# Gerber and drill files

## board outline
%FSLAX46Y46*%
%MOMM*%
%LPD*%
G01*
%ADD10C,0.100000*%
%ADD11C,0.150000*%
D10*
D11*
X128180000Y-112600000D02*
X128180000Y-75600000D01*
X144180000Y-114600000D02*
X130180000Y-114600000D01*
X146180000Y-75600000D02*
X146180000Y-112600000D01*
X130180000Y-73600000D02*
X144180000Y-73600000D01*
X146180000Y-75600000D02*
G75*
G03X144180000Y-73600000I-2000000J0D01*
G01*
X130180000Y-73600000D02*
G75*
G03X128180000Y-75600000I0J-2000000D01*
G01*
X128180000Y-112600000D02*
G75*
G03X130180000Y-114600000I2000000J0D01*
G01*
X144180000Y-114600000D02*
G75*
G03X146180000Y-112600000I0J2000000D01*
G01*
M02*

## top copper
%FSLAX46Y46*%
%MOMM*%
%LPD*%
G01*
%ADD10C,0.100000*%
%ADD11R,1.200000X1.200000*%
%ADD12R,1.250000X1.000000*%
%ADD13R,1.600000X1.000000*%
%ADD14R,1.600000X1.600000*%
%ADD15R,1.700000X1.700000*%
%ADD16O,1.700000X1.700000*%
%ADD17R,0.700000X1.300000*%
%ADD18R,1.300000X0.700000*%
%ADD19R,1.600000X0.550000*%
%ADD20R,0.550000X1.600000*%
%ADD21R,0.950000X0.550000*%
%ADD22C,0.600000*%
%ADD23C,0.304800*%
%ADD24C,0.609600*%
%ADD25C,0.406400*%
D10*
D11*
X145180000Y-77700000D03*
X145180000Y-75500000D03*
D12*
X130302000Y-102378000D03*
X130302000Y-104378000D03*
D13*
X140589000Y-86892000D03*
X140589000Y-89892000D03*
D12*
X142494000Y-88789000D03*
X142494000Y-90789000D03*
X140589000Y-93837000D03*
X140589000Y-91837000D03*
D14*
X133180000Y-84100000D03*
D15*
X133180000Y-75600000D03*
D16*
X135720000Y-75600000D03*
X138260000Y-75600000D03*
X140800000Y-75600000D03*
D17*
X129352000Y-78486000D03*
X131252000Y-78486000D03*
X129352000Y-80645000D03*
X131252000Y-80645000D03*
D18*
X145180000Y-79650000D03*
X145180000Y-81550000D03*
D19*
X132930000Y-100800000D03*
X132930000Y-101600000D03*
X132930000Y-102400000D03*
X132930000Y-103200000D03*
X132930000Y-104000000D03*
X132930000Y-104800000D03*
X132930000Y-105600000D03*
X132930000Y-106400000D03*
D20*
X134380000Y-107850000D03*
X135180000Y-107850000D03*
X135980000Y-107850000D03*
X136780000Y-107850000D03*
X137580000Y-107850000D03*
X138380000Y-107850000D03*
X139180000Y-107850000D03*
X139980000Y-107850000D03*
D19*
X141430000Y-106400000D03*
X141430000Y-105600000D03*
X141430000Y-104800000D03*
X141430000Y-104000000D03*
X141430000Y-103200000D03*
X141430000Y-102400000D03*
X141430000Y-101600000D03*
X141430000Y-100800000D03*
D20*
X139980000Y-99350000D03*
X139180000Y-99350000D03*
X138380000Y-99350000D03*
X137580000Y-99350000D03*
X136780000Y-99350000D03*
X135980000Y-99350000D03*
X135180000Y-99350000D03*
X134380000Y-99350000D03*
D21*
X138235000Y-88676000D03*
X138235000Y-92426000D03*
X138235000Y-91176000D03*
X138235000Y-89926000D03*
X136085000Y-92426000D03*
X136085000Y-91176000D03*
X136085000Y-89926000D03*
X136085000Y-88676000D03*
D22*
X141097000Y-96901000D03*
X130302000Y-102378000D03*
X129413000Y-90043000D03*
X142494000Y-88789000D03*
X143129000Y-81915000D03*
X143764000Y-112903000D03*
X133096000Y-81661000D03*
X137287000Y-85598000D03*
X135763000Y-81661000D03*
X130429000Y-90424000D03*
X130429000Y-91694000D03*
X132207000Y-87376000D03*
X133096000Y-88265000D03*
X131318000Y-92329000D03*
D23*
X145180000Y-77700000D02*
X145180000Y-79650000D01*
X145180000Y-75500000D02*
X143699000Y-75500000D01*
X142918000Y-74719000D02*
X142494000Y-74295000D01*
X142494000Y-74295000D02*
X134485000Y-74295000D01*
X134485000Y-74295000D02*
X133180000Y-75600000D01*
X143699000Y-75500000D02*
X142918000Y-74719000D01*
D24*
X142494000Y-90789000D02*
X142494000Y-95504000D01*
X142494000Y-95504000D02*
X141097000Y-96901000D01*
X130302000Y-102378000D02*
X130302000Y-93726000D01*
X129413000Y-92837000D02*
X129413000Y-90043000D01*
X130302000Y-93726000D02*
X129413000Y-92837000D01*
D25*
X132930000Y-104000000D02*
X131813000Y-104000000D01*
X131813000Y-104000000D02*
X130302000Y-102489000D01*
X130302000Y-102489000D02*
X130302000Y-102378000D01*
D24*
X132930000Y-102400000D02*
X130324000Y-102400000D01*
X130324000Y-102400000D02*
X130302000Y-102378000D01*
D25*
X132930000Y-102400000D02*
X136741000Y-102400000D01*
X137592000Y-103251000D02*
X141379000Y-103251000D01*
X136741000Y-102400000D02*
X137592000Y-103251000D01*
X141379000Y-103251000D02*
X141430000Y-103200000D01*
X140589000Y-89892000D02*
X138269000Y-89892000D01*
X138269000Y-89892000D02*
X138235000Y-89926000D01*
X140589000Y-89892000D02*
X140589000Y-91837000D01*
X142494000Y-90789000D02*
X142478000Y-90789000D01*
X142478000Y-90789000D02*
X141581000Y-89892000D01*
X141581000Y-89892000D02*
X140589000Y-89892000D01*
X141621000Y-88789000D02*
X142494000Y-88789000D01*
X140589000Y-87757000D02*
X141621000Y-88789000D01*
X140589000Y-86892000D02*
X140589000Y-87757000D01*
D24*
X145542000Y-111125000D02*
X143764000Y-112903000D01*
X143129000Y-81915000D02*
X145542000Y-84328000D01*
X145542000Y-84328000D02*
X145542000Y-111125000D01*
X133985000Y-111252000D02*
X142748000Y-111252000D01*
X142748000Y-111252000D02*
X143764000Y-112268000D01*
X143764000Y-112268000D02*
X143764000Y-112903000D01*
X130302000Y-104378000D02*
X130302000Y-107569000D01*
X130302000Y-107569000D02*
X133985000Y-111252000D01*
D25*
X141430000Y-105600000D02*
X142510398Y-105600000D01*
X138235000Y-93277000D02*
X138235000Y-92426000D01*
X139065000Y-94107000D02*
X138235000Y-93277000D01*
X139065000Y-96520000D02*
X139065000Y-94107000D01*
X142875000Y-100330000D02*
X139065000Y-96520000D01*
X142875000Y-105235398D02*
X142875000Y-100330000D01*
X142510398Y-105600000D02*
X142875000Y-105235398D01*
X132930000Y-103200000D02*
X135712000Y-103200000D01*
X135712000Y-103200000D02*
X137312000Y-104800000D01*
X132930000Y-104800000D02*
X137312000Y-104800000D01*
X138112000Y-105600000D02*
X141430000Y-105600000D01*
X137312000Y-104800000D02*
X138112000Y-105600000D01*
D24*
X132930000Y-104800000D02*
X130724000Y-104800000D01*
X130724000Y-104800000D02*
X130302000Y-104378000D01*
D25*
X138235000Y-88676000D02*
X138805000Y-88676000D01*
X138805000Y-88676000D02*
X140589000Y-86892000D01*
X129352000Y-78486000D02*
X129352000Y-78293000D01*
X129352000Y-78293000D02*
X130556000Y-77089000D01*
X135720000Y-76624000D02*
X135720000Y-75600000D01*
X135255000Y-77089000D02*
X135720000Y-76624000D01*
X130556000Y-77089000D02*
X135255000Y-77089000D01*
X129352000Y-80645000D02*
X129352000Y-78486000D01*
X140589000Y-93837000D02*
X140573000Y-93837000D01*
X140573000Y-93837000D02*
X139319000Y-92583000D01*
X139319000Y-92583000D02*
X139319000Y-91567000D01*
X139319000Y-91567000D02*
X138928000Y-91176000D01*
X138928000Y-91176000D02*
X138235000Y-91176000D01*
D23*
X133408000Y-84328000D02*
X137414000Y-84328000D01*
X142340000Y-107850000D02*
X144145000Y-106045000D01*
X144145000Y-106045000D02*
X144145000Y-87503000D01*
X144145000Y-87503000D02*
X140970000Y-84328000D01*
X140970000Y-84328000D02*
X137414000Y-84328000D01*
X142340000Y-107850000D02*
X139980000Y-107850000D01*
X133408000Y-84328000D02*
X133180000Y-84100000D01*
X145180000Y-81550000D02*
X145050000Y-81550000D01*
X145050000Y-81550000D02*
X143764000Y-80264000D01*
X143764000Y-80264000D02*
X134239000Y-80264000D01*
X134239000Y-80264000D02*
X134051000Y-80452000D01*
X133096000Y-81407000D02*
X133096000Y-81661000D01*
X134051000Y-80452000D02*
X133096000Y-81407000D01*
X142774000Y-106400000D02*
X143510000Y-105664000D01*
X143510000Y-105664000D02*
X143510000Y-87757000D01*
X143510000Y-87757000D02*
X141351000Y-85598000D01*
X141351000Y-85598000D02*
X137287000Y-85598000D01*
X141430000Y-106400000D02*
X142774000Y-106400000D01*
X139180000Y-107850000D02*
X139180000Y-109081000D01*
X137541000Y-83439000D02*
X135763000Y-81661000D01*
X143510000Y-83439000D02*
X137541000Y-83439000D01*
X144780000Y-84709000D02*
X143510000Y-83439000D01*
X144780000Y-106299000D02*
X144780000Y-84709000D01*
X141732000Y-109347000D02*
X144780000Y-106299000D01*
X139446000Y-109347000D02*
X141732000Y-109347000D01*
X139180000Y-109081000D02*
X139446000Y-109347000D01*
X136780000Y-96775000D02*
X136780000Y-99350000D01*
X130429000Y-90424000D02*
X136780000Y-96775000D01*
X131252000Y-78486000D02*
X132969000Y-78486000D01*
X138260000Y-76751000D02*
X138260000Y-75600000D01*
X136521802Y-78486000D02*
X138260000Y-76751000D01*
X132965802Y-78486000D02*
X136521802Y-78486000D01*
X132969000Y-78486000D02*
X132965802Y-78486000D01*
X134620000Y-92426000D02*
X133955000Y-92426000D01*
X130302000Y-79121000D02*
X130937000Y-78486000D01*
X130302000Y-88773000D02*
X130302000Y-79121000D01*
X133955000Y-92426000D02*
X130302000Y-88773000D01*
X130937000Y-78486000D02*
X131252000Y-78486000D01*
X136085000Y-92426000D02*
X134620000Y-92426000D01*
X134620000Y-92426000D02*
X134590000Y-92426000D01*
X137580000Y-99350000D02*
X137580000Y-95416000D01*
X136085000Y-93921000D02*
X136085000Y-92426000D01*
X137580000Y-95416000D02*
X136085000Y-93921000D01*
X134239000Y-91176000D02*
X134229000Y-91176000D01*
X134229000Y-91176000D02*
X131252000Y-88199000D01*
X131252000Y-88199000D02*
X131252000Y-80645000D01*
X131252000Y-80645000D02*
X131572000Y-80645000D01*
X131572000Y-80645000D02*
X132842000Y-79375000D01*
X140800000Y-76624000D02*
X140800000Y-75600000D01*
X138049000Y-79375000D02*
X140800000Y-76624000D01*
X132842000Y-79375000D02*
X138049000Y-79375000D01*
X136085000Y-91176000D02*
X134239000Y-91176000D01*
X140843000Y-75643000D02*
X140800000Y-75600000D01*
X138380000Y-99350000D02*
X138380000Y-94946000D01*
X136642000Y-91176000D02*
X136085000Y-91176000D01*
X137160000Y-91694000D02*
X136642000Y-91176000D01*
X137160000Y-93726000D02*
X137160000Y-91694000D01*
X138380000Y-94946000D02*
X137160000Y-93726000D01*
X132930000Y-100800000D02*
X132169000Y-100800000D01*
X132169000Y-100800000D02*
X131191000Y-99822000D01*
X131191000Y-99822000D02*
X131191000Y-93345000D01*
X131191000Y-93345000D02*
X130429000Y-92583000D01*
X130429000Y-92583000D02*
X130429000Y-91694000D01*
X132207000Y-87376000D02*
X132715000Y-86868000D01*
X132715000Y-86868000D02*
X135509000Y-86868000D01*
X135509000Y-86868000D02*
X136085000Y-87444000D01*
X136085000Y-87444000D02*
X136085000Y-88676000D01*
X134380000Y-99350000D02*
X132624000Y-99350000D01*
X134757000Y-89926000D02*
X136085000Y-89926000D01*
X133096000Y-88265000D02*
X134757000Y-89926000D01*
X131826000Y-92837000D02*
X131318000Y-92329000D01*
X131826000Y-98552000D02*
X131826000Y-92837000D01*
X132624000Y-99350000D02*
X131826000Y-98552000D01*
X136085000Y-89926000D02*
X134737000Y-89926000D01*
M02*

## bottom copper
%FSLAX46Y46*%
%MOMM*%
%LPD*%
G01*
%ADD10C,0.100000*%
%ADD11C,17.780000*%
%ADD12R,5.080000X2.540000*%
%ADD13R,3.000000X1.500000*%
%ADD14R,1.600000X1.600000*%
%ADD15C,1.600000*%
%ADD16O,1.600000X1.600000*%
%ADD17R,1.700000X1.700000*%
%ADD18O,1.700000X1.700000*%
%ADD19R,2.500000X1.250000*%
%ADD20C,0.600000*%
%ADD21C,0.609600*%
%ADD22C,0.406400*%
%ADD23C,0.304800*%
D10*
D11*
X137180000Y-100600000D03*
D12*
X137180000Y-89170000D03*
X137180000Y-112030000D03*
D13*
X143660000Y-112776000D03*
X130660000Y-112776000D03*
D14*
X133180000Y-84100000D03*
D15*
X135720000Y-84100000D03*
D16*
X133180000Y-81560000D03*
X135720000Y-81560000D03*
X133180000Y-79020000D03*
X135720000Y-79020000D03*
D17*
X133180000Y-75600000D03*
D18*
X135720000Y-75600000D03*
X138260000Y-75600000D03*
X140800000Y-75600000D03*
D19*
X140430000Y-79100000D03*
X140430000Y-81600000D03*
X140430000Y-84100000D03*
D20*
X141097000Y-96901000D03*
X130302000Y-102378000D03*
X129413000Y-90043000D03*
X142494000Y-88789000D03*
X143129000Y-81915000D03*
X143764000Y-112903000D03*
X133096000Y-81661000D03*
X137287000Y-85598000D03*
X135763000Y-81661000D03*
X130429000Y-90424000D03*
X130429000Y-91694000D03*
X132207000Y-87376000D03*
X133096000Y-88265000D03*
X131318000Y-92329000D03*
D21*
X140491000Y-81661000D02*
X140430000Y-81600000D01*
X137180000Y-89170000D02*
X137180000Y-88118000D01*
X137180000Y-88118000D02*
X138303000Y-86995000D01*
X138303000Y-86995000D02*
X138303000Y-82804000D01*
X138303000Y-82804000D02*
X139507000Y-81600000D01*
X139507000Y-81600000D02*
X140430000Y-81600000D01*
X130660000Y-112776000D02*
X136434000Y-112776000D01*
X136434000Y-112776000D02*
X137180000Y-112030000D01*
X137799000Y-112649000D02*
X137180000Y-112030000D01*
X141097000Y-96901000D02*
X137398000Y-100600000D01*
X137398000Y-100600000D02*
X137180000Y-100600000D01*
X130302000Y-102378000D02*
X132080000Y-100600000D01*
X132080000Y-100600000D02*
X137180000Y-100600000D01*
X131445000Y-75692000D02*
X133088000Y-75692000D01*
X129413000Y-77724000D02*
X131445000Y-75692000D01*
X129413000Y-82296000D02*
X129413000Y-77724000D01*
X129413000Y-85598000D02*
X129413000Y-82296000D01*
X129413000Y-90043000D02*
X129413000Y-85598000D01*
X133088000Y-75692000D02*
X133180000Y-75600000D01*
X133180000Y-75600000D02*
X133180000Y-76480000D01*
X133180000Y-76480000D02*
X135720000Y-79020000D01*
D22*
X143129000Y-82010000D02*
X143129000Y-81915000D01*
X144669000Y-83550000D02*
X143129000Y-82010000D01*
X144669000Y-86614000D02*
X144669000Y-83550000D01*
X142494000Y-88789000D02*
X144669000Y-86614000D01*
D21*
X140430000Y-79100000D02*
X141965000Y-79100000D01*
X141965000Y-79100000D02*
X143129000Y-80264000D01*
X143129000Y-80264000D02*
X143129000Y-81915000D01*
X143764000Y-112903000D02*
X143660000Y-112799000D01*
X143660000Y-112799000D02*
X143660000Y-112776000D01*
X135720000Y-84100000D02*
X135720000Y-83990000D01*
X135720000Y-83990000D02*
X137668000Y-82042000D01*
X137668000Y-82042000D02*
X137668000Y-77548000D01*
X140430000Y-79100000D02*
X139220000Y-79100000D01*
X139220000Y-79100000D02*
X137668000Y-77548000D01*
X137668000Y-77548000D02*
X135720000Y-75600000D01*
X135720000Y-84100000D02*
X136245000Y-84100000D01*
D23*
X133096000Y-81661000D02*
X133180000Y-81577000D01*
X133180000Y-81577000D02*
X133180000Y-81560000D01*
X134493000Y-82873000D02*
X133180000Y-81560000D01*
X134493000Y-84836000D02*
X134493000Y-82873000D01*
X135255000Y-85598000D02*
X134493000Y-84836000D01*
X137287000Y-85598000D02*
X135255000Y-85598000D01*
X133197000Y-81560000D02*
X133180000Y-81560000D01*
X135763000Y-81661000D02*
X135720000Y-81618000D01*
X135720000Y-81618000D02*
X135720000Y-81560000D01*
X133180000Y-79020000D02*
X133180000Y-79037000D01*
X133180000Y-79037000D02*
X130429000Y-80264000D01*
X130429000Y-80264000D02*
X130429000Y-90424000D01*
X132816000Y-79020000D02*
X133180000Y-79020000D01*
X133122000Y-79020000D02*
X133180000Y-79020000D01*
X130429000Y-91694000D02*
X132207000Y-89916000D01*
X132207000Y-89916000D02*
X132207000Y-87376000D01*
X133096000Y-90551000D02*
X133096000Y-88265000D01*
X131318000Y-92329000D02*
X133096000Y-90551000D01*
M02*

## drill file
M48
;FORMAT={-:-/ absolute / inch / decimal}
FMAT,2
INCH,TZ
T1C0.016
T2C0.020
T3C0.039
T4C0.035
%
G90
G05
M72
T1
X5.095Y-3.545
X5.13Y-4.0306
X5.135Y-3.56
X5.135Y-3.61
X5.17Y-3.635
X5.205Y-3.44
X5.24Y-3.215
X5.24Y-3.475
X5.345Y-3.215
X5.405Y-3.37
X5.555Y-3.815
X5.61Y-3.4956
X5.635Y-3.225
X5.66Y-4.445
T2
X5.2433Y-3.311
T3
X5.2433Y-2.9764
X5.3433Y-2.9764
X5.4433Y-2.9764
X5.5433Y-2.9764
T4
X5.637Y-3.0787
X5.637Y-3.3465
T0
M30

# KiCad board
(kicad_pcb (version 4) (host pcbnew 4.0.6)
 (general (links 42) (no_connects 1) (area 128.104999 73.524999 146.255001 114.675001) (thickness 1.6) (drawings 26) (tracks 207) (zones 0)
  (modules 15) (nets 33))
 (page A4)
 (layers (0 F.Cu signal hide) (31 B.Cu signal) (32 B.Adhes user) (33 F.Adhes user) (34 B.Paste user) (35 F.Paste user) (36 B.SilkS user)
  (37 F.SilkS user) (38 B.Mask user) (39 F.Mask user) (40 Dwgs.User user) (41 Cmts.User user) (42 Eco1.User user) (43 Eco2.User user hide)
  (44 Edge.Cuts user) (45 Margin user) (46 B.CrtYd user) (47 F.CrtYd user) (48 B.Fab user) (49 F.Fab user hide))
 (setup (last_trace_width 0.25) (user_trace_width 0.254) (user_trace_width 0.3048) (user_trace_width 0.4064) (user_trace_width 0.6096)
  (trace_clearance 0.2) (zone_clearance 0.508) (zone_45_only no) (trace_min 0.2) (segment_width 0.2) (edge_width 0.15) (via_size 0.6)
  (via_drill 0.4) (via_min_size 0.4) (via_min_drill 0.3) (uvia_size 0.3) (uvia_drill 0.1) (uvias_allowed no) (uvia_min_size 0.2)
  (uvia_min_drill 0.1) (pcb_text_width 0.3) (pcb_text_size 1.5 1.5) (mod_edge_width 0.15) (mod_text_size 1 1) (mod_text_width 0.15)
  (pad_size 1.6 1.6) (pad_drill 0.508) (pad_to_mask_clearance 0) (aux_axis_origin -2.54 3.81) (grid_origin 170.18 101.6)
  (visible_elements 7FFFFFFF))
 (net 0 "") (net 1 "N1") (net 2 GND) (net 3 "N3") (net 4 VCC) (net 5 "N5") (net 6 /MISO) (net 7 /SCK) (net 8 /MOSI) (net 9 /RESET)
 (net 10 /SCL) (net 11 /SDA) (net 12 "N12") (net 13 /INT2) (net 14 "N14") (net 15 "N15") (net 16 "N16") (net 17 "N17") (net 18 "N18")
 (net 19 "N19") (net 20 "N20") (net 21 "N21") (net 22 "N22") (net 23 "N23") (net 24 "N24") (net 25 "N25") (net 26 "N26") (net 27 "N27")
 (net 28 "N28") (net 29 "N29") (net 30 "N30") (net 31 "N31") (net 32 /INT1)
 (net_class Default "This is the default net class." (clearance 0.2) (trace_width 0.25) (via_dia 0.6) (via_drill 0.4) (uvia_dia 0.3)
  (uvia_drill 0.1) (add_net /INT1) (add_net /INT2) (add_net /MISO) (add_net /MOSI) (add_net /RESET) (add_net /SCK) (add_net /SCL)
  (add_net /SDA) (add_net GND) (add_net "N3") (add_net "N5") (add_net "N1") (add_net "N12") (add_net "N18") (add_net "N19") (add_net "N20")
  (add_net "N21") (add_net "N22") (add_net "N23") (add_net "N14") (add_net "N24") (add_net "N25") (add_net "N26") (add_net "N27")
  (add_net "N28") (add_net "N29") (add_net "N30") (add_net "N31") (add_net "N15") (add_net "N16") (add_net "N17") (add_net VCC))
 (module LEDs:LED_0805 (layer F.Cu) (at 145.18 76.6 270)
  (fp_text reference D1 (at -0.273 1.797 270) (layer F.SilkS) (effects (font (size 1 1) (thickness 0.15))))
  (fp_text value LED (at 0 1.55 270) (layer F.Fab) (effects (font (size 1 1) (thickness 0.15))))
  (pad 2 smd rect (at 1.1 0 90) (size 1.2 1.2) (layers F.Cu F.Paste F.Mask) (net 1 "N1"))
  (pad 1 smd rect (at -1.1 0 90) (size 1.2 1.2) (layers F.Cu F.Paste F.Mask) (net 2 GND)))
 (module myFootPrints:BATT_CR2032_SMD (layer B.Cu) (at 137.18 100.6 270)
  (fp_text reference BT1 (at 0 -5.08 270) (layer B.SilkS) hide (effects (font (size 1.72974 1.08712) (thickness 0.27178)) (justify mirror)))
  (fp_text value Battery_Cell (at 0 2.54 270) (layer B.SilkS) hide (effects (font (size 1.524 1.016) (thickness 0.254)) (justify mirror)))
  (pad 2 smd circle (at 0 0 270) (size 17.78 17.78) (layers B.Cu B.Paste B.Mask) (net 2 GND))
  (pad 1 smd rect (at -11.43 0 270) (size 2.54 5.08) (layers B.Cu B.Paste B.Mask) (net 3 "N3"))
  (pad 1 smd rect (at 11.43 0 270) (size 2.54 5.08) (layers B.Cu B.Paste B.Mask) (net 3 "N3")))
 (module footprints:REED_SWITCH (layer B.Cu) (at 137.16 112.776 180)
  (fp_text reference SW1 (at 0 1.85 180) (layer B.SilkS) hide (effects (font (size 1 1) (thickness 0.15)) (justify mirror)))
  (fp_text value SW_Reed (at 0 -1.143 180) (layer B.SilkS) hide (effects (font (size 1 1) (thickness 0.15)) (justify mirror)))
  (pad 1 smd rect (at -6.5 0 180) (size 3 1.5) (layers B.Cu B.Paste B.Mask) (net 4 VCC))
  (pad 2 smd rect (at 6.5 0 180) (size 3 1.5) (layers B.Cu B.Paste B.Mask) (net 3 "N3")))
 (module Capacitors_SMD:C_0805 (layer F.Cu) (at 130.302 103.378 270)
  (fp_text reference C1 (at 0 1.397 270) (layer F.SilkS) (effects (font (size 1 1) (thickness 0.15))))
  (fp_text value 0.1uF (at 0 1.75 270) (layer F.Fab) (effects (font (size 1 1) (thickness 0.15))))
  (pad 1 smd rect (at -1 0 270) (size 1 1.25) (layers F.Cu F.Paste F.Mask) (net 2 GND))
  (pad 2 smd rect (at 1 0 270) (size 1 1.25) (layers F.Cu F.Paste F.Mask) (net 4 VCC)))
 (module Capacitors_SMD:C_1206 (layer F.Cu) (at 140.589 88.392 270)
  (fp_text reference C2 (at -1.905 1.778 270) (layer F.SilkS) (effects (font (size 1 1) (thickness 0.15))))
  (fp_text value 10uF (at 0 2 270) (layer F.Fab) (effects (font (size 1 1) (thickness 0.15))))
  (pad 1 smd rect (at -1.5 0 270) (size 1 1.6) (layers F.Cu F.Paste F.Mask) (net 4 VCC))
  (pad 2 smd rect (at 1.5 0 270) (size 1 1.6) (layers F.Cu F.Paste F.Mask) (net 2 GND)))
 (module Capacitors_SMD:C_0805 (layer F.Cu) (at 142.494 89.789 270)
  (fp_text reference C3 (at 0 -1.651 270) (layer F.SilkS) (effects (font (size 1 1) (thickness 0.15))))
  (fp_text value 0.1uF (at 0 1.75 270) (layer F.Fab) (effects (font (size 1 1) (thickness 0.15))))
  (pad 1 smd rect (at -1 0 270) (size 1 1.25) (layers F.Cu F.Paste F.Mask) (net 4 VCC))
  (pad 2 smd rect (at 1 0 270) (size 1 1.25) (layers F.Cu F.Paste F.Mask) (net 2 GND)))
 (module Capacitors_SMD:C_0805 (layer F.Cu) (at 140.589 92.837 90)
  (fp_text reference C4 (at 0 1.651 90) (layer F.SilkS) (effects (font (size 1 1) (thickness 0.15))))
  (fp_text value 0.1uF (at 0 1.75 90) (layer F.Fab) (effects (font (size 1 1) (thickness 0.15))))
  (pad 1 smd rect (at -1 0 90) (size 1 1.25) (layers F.Cu F.Paste F.Mask) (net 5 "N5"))
  (pad 2 smd rect (at 1 0 90) (size 1 1.25) (layers F.Cu F.Paste F.Mask) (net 2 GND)))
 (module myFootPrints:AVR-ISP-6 (layer B.Cu) (at 133.18 84.1)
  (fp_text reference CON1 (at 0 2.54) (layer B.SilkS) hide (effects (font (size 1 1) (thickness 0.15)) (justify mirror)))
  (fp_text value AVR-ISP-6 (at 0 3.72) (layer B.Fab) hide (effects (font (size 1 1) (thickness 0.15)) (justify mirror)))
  (pad 1 thru_hole rect (at 0 0) (size 1.6 1.6) (drill 0.508) (layers *.Cu B.Mask) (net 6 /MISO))
  (pad 2 smd circle (at 2.54 0) (size 1.6 1.6) (layers B.Cu B.Paste B.Mask) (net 4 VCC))
  (pad 3 smd oval (at 0 -2.54) (size 1.6 1.6) (layers B.Cu B.Paste B.Mask) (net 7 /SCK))
  (pad 4 smd oval (at 2.54 -2.54) (size 1.6 1.6) (layers B.Cu B.Paste B.Mask) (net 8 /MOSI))
  (pad 5 smd oval (at 0 -5.08) (size 1.6 1.6) (layers B.Cu B.Paste B.Mask) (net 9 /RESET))
  (pad 6 smd oval (at 2.54 -5.08) (size 1.6 1.6) (layers B.Cu B.Paste B.Mask) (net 2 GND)))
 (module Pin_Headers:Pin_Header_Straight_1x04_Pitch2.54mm (layer F.Cu) (at 133.18 75.6 90)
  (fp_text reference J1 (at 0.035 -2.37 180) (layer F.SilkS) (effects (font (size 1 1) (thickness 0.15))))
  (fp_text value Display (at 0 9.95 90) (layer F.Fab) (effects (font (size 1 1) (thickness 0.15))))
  (pad 1 thru_hole rect (at 0 0 90) (size 1.7 1.7) (drill 1) (layers *.Cu *.Mask) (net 2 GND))
  (pad 2 thru_hole oval (at 0 2.54 90) (size 1.7 1.7) (drill 1) (layers *.Cu *.Mask) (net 4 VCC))
  (pad 3 thru_hole oval (at 0 5.08 90) (size 1.7 1.7) (drill 1) (layers *.Cu *.Mask) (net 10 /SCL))
  (pad 4 thru_hole oval (at 0 7.62 90) (size 1.7 1.7) (drill 1) (layers *.Cu *.Mask) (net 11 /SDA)))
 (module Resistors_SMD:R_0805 (layer F.Cu) (at 130.302 78.486)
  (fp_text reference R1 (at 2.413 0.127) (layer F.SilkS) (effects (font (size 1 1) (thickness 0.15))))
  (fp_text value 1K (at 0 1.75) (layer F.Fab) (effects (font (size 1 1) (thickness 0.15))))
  (pad 1 smd rect (at -0.95 0) (size 0.7 1.3) (layers F.Cu F.Paste F.Mask) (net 4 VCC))
  (pad 2 smd rect (at 0.95 0) (size 0.7 1.3) (layers F.Cu F.Paste F.Mask) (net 10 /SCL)))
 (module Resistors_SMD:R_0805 (layer F.Cu) (at 130.302 80.645)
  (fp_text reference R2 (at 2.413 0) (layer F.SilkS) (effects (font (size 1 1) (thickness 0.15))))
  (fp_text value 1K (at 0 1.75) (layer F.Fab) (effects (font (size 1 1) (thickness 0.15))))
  (pad 1 smd rect (at -0.95 0) (size 0.7 1.3) (layers F.Cu F.Paste F.Mask) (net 4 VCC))
  (pad 2 smd rect (at 0.95 0) (size 0.7 1.3) (layers F.Cu F.Paste F.Mask) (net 11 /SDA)))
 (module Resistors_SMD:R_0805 (layer F.Cu) (at 145.18 80.6 270)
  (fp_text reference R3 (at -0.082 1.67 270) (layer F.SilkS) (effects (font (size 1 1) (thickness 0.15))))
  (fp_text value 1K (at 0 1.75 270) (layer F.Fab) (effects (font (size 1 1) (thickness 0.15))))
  (pad 1 smd rect (at -0.95 0 270) (size 0.7 1.3) (layers F.Cu F.Paste F.Mask) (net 1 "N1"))
  (pad 2 smd rect (at 0.95 0 270) (size 0.7 1.3) (layers F.Cu F.Paste F.Mask) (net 7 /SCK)))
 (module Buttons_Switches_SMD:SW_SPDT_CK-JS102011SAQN (layer B.Cu) (at 143.18 81.6 270)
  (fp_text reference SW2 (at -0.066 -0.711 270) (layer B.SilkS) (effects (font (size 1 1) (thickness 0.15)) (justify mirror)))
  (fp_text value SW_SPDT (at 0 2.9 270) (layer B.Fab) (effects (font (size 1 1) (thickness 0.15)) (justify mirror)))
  (pad 1 smd rect (at -2.5 2.75 270) (size 1.25 2.5) (layers B.Cu B.Paste B.Mask) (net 4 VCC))
  (pad 2 smd rect (at 0 2.75 270) (size 1.25 2.5) (layers B.Cu B.Paste B.Mask) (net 3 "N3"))
  (pad 3 smd rect (at 2.5 2.75 270) (size 1.25 2.5) (layers B.Cu B.Paste B.Mask) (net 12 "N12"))
  (pad "" np_thru_hole circle (at -3.4 0 270) (size 0.9 0.9) (drill 0.9) (layers *.Cu *.Mask))
  (pad "" np_thru_hole circle (at 3.4 0 270) (size 0.9 0.9) (drill 0.9) (layers *.Cu *.Mask)))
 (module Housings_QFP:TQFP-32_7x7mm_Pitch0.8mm (layer F.Cu) (at 137.18 103.6)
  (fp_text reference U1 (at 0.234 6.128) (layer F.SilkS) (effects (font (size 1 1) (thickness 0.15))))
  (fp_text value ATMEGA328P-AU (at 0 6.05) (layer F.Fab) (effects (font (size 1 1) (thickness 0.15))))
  (pad 1 smd rect (at -4.25 -2.8) (size 1.6 0.55) (layers F.Cu F.Paste F.Mask) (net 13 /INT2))
  (pad 2 smd rect (at -4.25 -2) (size 1.6 0.55) (layers F.Cu F.Paste F.Mask) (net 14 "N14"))
  (pad 3 smd rect (at -4.25 -1.2) (size 1.6 0.55) (layers F.Cu F.Paste F.Mask) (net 2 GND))
  (pad 4 smd rect (at -4.25 -0.4) (size 1.6 0.55) (layers F.Cu F.Paste F.Mask) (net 4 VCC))
  (pad 5 smd rect (at -4.25 0.4) (size 1.6 0.55) (layers F.Cu F.Paste F.Mask) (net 2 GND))
  (pad 6 smd rect (at -4.25 1.2) (size 1.6 0.55) (layers F.Cu F.Paste F.Mask) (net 4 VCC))
  (pad 7 smd rect (at -4.25 2) (size 1.6 0.55) (layers F.Cu F.Paste F.Mask) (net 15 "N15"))
  (pad 8 smd rect (at -4.25 2.8) (size 1.6 0.55) (layers F.Cu F.Paste F.Mask) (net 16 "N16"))
  (pad 9 smd rect (at -2.8 4.25 90) (size 1.6 0.55) (layers F.Cu F.Paste F.Mask) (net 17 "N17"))
  (pad 10 smd rect (at -2 4.25 90) (size 1.6 0.55) (layers F.Cu F.Paste F.Mask) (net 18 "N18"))
  (pad 11 smd rect (at -1.2 4.25 90) (size 1.6 0.55) (layers F.Cu F.Paste F.Mask) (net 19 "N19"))
  (pad 12 smd rect (at -0.4 4.25 90) (size 1.6 0.55) (layers F.Cu F.Paste F.Mask) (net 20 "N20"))
  (pad 13 smd rect (at 0.4 4.25 90) (size 1.6 0.55) (layers F.Cu F.Paste F.Mask) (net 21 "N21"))
  (pad 14 smd rect (at 1.2 4.25 90) (size 1.6 0.55) (layers F.Cu F.Paste F.Mask) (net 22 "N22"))
  (pad 15 smd rect (at 2 4.25 90) (size 1.6 0.55) (layers F.Cu F.Paste F.Mask) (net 8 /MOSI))
  (pad 16 smd rect (at 2.8 4.25 90) (size 1.6 0.55) (layers F.Cu F.Paste F.Mask) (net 6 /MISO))
  (pad 17 smd rect (at 4.25 2.8) (size 1.6 0.55) (layers F.Cu F.Paste F.Mask) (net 7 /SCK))
  (pad 18 smd rect (at 4.25 2) (size 1.6 0.55) (layers F.Cu F.Paste F.Mask) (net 4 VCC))
  (pad 19 smd rect (at 4.25 1.2) (size 1.6 0.55) (layers F.Cu F.Paste F.Mask) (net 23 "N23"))
  (pad 20 smd rect (at 4.25 0.4) (size 1.6 0.55) (layers F.Cu F.Paste F.Mask) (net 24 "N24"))
  (pad 21 smd rect (at 4.25 -0.4) (size 1.6 0.55) (layers F.Cu F.Paste F.Mask) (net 2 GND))
  (pad 22 smd rect (at 4.25 -1.2) (size 1.6 0.55) (layers F.Cu F.Paste F.Mask) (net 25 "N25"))
  (pad 23 smd rect (at 4.25 -2) (size 1.6 0.55) (layers F.Cu F.Paste F.Mask) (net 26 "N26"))
  (pad 24 smd rect (at 4.25 -2.8) (size 1.6 0.55) (layers F.Cu F.Paste F.Mask) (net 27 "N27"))
  (pad 25 smd rect (at 2.8 -4.25 90) (size 1.6 0.55) (layers F.Cu F.Paste F.Mask) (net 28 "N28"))
  (pad 26 smd rect (at 2 -4.25 90) (size 1.6 0.55) (layers F.Cu F.Paste F.Mask) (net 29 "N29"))
  (pad 27 smd rect (at 1.2 -4.25 90) (size 1.6 0.55) (layers F.Cu F.Paste F.Mask) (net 11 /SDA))
  (pad 28 smd rect (at 0.4 -4.25 90) (size 1.6 0.55) (layers F.Cu F.Paste F.Mask) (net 10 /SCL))
  (pad 29 smd rect (at -0.4 -4.25 90) (size 1.6 0.55) (layers F.Cu F.Paste F.Mask) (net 9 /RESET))
  (pad 30 smd rect (at -1.2 -4.25 90) (size 1.6 0.55) (layers F.Cu F.Paste F.Mask) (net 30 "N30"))
  (pad 31 smd rect (at -2 -4.25 90) (size 1.6 0.55) (layers F.Cu F.Paste F.Mask) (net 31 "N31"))
  (pad 32 smd rect (at -2.8 -4.25 90) (size 1.6 0.55) (layers F.Cu F.Paste F.Mask) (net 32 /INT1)))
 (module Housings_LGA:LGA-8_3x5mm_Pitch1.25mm (layer F.Cu) (at 137.16 90.551 180)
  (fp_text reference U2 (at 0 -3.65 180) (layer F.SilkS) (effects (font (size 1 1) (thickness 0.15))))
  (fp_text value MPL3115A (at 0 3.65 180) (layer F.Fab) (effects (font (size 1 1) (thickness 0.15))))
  (pad 4 smd rect (at -1.075 1.875 180) (size 0.95 0.55) (layers F.Cu F.Paste F.Mask) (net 4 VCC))
  (pad 1 smd rect (at -1.075 -1.875 180) (size 0.95 0.55) (layers F.Cu F.Paste F.Mask) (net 4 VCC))
  (pad 2 smd rect (at -1.075 -0.625 180) (size 0.95 0.55) (layers F.Cu F.Paste F.Mask) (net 5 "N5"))
  (pad 3 smd rect (at -1.075 0.625 180) (size 0.95 0.55) (layers F.Cu F.Paste F.Mask) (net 2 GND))
  (pad 8 smd rect (at 1.075 -1.875 180) (size 0.95 0.55) (layers F.Cu F.Paste F.Mask) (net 10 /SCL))
  (pad 7 smd rect (at 1.075 -0.625 180) (size 0.95 0.55) (layers F.Cu F.Paste F.Mask) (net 11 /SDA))
  (pad 6 smd rect (at 1.075 0.625 180) (size 0.95 0.55) (layers F.Cu F.Paste F.Mask) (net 32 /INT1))
  (pad 5 smd rect (at 1.075 1.875 180) (size 0.95 0.55) (layers F.Cu F.Paste F.Mask) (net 13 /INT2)))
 (gr_line (start 128.18 112.6) (end 128.18 75.6) (angle 90) (layer Edge.Cuts) (width 0.15))
 (gr_line (start 144.18 114.6) (end 130.18 114.6) (angle 90) (layer Edge.Cuts) (width 0.15))
 (gr_line (start 146.18 75.6) (end 146.18 112.6) (angle 90) (layer Edge.Cuts) (width 0.15))
 (gr_line (start 130.18 73.6) (end 144.18 73.6) (angle 90) (layer Edge.Cuts) (width 0.15))
 (gr_arc (start 144.18 75.6) (end 144.18 73.6) (angle 90) (layer Edge.Cuts) (width 0.15))
 (gr_arc (start 130.18 75.6) (end 128.18 75.6) (angle 90) (layer Edge.Cuts) (width 0.15))
 (gr_arc (start 130.18 112.6) (end 130.18 114.6) (angle 90) (layer Edge.Cuts) (width 0.15))
 (gr_arc (start 144.18 112.6) (end 146.18 112.6) (angle 90) (layer Edge.Cuts) (width 0.15))
 (segment (start 140.491 81.661) (end 140.43 81.6) (width 0.6096) (layer B.Cu) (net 3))
 (segment (start 137.18 89.17) (end 137.18 88.118) (width 0.6096) (layer B.Cu) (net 3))
 (segment (start 137.18 88.118) (end 138.303 86.995) (width 0.6096) (layer B.Cu) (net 3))
 (segment (start 138.303 86.995) (end 138.303 82.804) (width 0.6096) (layer B.Cu) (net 3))
 (segment (start 138.303 82.804) (end 139.507 81.6) (width 0.6096) (layer B.Cu) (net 3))
 (segment (start 139.507 81.6) (end 140.43 81.6) (width 0.6096) (layer B.Cu) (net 3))
 (segment (start 130.66 112.776) (end 136.434 112.776) (width 0.6096) (layer B.Cu) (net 3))
 (segment (start 136.434 112.776) (end 137.18 112.03) (width 0.6096) (layer B.Cu) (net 3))
 (segment (start 137.799 112.649) (end 137.18 112.03) (width 0.6096) (layer B.Cu) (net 3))
 (segment (start 145.18 77.7) (end 145.18 79.65) (width 0.3048) (layer F.Cu) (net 1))
 (segment (start 145.18 75.5) (end 143.699 75.5) (width 0.3048) (layer F.Cu) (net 2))
 (segment (start 142.918 74.719) (end 142.494 74.295) (width 0.3048) (layer F.Cu) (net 2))
 (segment (start 142.494 74.295) (end 134.485 74.295) (width 0.3048) (layer F.Cu) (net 2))
 (segment (start 134.485 74.295) (end 133.18 75.6) (width 0.3048) (layer F.Cu) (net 2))
 (segment (start 143.699 75.5) (end 142.918 74.719) (width 0.3048) (layer F.Cu) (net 2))
 (segment (start 142.494 90.789) (end 142.494 95.504) (width 0.6096) (layer F.Cu) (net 2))
 (segment (start 141.097 96.901) (end 137.398 100.6) (width 0.6096) (layer B.Cu) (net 2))
 (via (at 141.097 96.901) (size 0.6) (drill 0.4) (layers F.Cu B.Cu) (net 2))
 (segment (start 142.494 95.504) (end 141.097 96.901) (width 0.6096) (layer F.Cu) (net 2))
 (segment (start 137.398 100.6) (end 137.18 100.6) (width 0.6096) (layer B.Cu) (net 2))
 (via (at 130.302 102.378) (size 0.6) (drill 0.4) (layers F.Cu B.Cu) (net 2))
 (segment (start 130.302 102.378) (end 132.08 100.6) (width 0.6096) (layer B.Cu) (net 2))
 (segment (start 132.08 100.6) (end 137.18 100.6) (width 0.6096) (layer B.Cu) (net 2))
 (segment (start 130.302 102.378) (end 130.302 93.726) (width 0.6096) (layer F.Cu) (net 2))
 (segment (start 131.445 75.692) (end 133.088 75.692) (width 0.6096) (layer B.Cu) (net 2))
 (segment (start 129.413 77.724) (end 131.445 75.692) (width 0.6096) (layer B.Cu) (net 2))
 (segment (start 129.413 82.296) (end 129.413 77.724) (width 0.6096) (layer B.Cu) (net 2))
 (segment (start 129.413 85.598) (end 129.413 82.296) (width 0.6096) (layer B.Cu) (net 2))
 (segment (start 129.413 90.043) (end 129.413 85.598) (width 0.6096) (layer B.Cu) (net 2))
 (via (at 129.413 90.043) (size 0.6) (drill 0.4) (layers F.Cu B.Cu) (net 2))
 (segment (start 129.413 92.837) (end 129.413 90.043) (width 0.6096) (layer F.Cu) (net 2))
 (segment (start 130.302 93.726) (end 129.413 92.837) (width 0.6096) (layer F.Cu) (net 2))
 (segment (start 133.088 75.692) (end 133.18 75.6) (width 0.6096) (layer B.Cu) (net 2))
 (segment (start 132.93 104) (end 131.813 104) (width 0.4064) (layer F.Cu) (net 2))
 (segment (start 131.813 104) (end 130.302 102.489) (width 0.4064) (layer F.Cu) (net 2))
 (segment (start 130.302 102.489) (end 130.302 102.378) (width 0.4064) (layer F.Cu) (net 2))
 (segment (start 132.93 102.4) (end 130.324 102.4) (width 0.6096) (layer F.Cu) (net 2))
 (segment (start 130.324 102.4) (end 130.302 102.378) (width 0.6096) (layer F.Cu) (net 2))
 (segment (start 132.93 102.4) (end 136.741 102.4) (width 0.4064) (layer F.Cu) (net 2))
 (segment (start 137.592 103.251) (end 141.379 103.251) (width 0.4064) (layer F.Cu) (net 2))
 (segment (start 136.741 102.4) (end 137.592 103.251) (width 0.4064) (layer F.Cu) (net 2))
 (segment (start 141.379 103.251) (end 141.43 103.2) (width 0.4064) (layer F.Cu) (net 2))
 (segment (start 140.589 89.892) (end 138.269 89.892) (width 0.4064) (layer F.Cu) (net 2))
 (segment (start 138.269 89.892) (end 138.235 89.926) (width 0.4064) (layer F.Cu) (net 2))
 (segment (start 140.589 89.892) (end 140.589 91.837) (width 0.4064) (layer F.Cu) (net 2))
 (segment (start 142.494 90.789) (end 142.478 90.789) (width 0.4064) (layer F.Cu) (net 2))
 (segment (start 142.478 90.789) (end 141.581 89.892) (width 0.4064) (layer F.Cu) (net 2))
 (segment (start 141.581 89.892) (end 140.589 89.892) (width 0.4064) (layer F.Cu) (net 2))
 (segment (start 133.18 75.6) (end 133.18 76.48) (width 0.6096) (layer B.Cu) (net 2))
 (segment (start 133.18 76.48) (end 135.72 79.02) (width 0.6096) (layer B.Cu) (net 2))
 (via (at 142.494 88.789) (size 0.6) (drill 0.4) (layers F.Cu B.Cu) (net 4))
 (segment (start 141.621 88.789) (end 142.494 88.789) (width 0.4064) (layer F.Cu) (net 4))
 (segment (start 140.589 87.757) (end 141.621 88.789) (width 0.4064) (layer F.Cu) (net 4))
 (segment (start 140.589 86.892) (end 140.589 87.757) (width 0.4064) (layer F.Cu) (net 4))
 (segment (start 143.129 82.01) (end 143.129 81.915) (width 0.4064) (layer B.Cu) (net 4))
 (segment (start 144.669 83.55) (end 143.129 82.01) (width 0.4064) (layer B.Cu) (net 4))
 (segment (start 144.669 86.614) (end 144.669 83.55) (width 0.4064) (layer B.Cu) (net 4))
 (segment (start 142.494 88.789) (end 144.669 86.614) (width 0.4064) (layer B.Cu) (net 4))
 (segment (start 140.43 79.1) (end 141.965 79.1) (width 0.6096) (layer B.Cu) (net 4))
 (segment (start 141.965 79.1) (end 143.129 80.264) (width 0.6096) (layer B.Cu) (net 4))
 (segment (start 143.129 80.264) (end 143.129 81.915) (width 0.6096) (layer B.Cu) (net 4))
 (segment (start 145.542 111.125) (end 143.764 112.903) (width 0.6096) (layer F.Cu) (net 4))
 (via (at 143.129 81.915) (size 0.6) (drill 0.4) (layers F.Cu B.Cu) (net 4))
 (segment (start 143.129 81.915) (end 145.542 84.328) (width 0.6096) (layer F.Cu) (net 4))
 (segment (start 145.542 84.328) (end 145.542 111.125) (width 0.6096) (layer F.Cu) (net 4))
 (segment (start 133.985 111.252) (end 142.748 111.252) (width 0.6096) (layer F.Cu) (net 4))
 (segment (start 142.748 111.252) (end 143.764 112.268) (width 0.6096) (layer F.Cu) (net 4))
 (segment (start 143.764 112.268) (end 143.764 112.903) (width 0.6096) (layer F.Cu) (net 4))
 (segment (start 130.302 104.378) (end 130.302 107.569) (width 0.6096) (layer F.Cu) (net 4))
 (segment (start 130.302 107.569) (end 133.985 111.252) (width 0.6096) (layer F.Cu) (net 4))
 (segment (start 143.764 112.903) (end 143.66 112.799) (width 0.6096) (layer B.Cu) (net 4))
 (via (at 143.764 112.903) (size 0.6) (drill 0.4) (layers F.Cu B.Cu) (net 4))
 (segment (start 143.66 112.799) (end 143.66 112.776) (width 0.6096) (layer B.Cu) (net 4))
 (segment (start 135.72 84.1) (end 135.72 83.99) (width 0.6096) (layer B.Cu) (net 4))
 (segment (start 135.72 83.99) (end 137.668 82.042) (width 0.6096) (layer B.Cu) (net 4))
 (segment (start 137.668 82.042) (end 137.668 77.548) (width 0.6096) (layer B.Cu) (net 4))
 (segment (start 140.43 79.1) (end 139.22 79.1) (width 0.6096) (layer B.Cu) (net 4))
 (segment (start 139.22 79.1) (end 137.668 77.548) (width 0.6096) (layer B.Cu) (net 4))
 (segment (start 137.668 77.548) (end 135.72 75.6) (width 0.6096) (layer B.Cu) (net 4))
 (segment (start 141.43 105.6) (end 142.510398 105.6) (width 0.4064) (layer F.Cu) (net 4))
 (segment (start 138.235 93.277) (end 138.235 92.426) (width 0.4064) (layer F.Cu) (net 4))
 (segment (start 139.065 94.107) (end 138.235 93.277) (width 0.4064) (layer F.Cu) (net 4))
 (segment (start 139.065 96.52) (end 139.065 94.107) (width 0.4064) (layer F.Cu) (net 4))
 (segment (start 142.875 100.33) (end 139.065 96.52) (width 0.4064) (layer F.Cu) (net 4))
 (segment (start 142.875 105.235398) (end 142.875 100.33) (width 0.4064) (layer F.Cu) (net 4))
 (segment (start 142.510398 105.6) (end 142.875 105.235398) (width 0.4064) (layer F.Cu) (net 4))
 (segment (start 132.93 103.2) (end 135.712 103.2) (width 0.4064) (layer F.Cu) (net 4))
 (segment (start 135.712 103.2) (end 137.312 104.8) (width 0.4064) (layer F.Cu) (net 4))
 (segment (start 132.93 104.8) (end 137.312 104.8) (width 0.4064) (layer F.Cu) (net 4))
 (segment (start 138.112 105.6) (end 141.43 105.6) (width 0.4064) (layer F.Cu) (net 4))
 (segment (start 137.312 104.8) (end 138.112 105.6) (width 0.4064) (layer F.Cu) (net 4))
 (segment (start 132.93 104.8) (end 130.724 104.8) (width 0.6096) (layer F.Cu) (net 4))
 (segment (start 130.724 104.8) (end 130.302 104.378) (width 0.6096) (layer F.Cu) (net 4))
 (segment (start 138.235 88.676) (end 138.805 88.676) (width 0.4064) (layer F.Cu) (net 4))
 (segment (start 138.805 88.676) (end 140.589 86.892) (width 0.4064) (layer F.Cu) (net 4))
 (segment (start 129.352 78.486) (end 129.352 78.293) (width 0.4064) (layer F.Cu) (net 4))
 (segment (start 129.352 78.293) (end 130.556 77.089) (width 0.4064) (layer F.Cu) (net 4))
 (segment (start 135.72 76.624) (end 135.72 75.6) (width 0.4064) (layer F.Cu) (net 4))
 (segment (start 135.255 77.089) (end 135.72 76.624) (width 0.4064) (layer F.Cu) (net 4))
 (segment (start 130.556 77.089) (end 135.255 77.089) (width 0.4064) (layer F.Cu) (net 4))
 (segment (start 129.352 80.645) (end 129.352 78.486) (width 0.4064) (layer F.Cu) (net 4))
 (segment (start 135.72 84.1) (end 136.245 84.1) (width 0.6096) (layer B.Cu) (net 4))
 (segment (start 140.589 93.837) (end 140.573 93.837) (width 0.4064) (layer F.Cu) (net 5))
 (segment (start 140.573 93.837) (end 139.319 92.583) (width 0.4064) (layer F.Cu) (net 5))
 (segment (start 139.319 92.583) (end 139.319 91.567) (width 0.4064) (layer F.Cu) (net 5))
 (segment (start 139.319 91.567) (end 138.928 91.176) (width 0.4064) (layer F.Cu) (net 5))
 (segment (start 138.928 91.176) (end 138.235 91.176) (width 0.4064) (layer F.Cu) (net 5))
 (segment (start 133.408 84.328) (end 137.414 84.328) (width 0.3048) (layer F.Cu) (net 6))
 (segment (start 142.34 107.85) (end 144.145 106.045) (width 0.3048) (layer F.Cu) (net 6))
 (segment (start 144.145 106.045) (end 144.145 87.503) (width 0.3048) (layer F.Cu) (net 6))
 (segment (start 144.145 87.503) (end 140.97 84.328) (width 0.3048) (layer F.Cu) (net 6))
 (segment (start 140.97 84.328) (end 137.414 84.328) (width 0.3048) (layer F.Cu) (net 6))
 (segment (start 142.34 107.85) (end 139.98 107.85) (width 0.3048) (layer F.Cu) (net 6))
 (segment (start 133.408 84.328) (end 133.18 84.1) (width 0.3048) (layer F.Cu) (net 6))
 (segment (start 145.18 81.55) (end 145.05 81.55) (width 0.3048) (layer F.Cu) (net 7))
 (segment (start 145.05 81.55) (end 143.764 80.264) (width 0.3048) (layer F.Cu) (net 7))
 (segment (start 143.764 80.264) (end 134.239 80.264) (width 0.3048) (layer F.Cu) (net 7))
 (segment (start 134.239 80.264) (end 134.051 80.452) (width 0.3048) (layer F.Cu) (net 7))
 (segment (start 133.096 81.661) (end 133.18 81.577) (width 0.3048) (layer B.Cu) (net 7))
 (via (at 133.096 81.661) (size 0.6) (drill 0.4) (layers F.Cu B.Cu) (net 7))
 (segment (start 133.096 81.407) (end 133.096 81.661) (width 0.3048) (layer F.Cu) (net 7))
 (segment (start 134.051 80.452) (end 133.096 81.407) (width 0.3048) (layer F.Cu) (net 7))
 (segment (start 133.18 81.577) (end 133.18 81.56) (width 0.3048) (layer B.Cu) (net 7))
 (via (at 137.287 85.598) (size 0.6) (drill 0.4) (layers F.Cu B.Cu) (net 7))
 (segment (start 142.774 106.4) (end 143.51 105.664) (width 0.3048) (layer F.Cu) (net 7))
 (segment (start 143.51 105.664) (end 143.51 87.757) (width 0.3048) (layer F.Cu) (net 7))
 (segment (start 143.51 87.757) (end 141.351 85.598) (width 0.3048) (layer F.Cu) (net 7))
 (segment (start 141.351 85.598) (end 137.287 85.598) (width 0.3048) (layer F.Cu) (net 7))
 (segment (start 141.43 106.4) (end 142.774 106.4) (width 0.3048) (layer F.Cu) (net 7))
 (segment (start 134.493 82.873) (end 133.18 81.56) (width 0.3048) (layer B.Cu) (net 7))
 (segment (start 134.493 84.836) (end 134.493 82.873) (width 0.3048) (layer B.Cu) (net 7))
 (segment (start 135.255 85.598) (end 134.493 84.836) (width 0.3048) (layer B.Cu) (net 7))
 (segment (start 137.287 85.598) (end 135.255 85.598) (width 0.3048) (layer B.Cu) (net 7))
 (segment (start 133.197 81.56) (end 133.18 81.56) (width 0.3048) (layer B.Cu) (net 7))
 (segment (start 139.18 107.85) (end 139.18 109.081) (width 0.3048) (layer F.Cu) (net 8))
 (segment (start 135.763 81.661) (end 135.72 81.618) (width 0.3048) (layer B.Cu) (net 8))
 (via (at 135.763 81.661) (size 0.6) (drill 0.4) (layers F.Cu B.Cu) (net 8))
 (segment (start 137.541 83.439) (end 135.763 81.661) (width 0.3048) (layer F.Cu) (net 8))
 (segment (start 143.51 83.439) (end 137.541 83.439) (width 0.3048) (layer F.Cu) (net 8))
 (segment (start 144.78 84.709) (end 143.51 83.439) (width 0.3048) (layer F.Cu) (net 8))
 (segment (start 144.78 106.299) (end 144.78 84.709) (width 0.3048) (layer F.Cu) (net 8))
 (segment (start 141.732 109.347) (end 144.78 106.299) (width 0.3048) (layer F.Cu) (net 8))
 (segment (start 139.446 109.347) (end 141.732 109.347) (width 0.3048) (layer F.Cu) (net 8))
 (segment (start 139.18 109.081) (end 139.446 109.347) (width 0.3048) (layer F.Cu) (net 8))
 (segment (start 135.72 81.618) (end 135.72 81.56) (width 0.3048) (layer B.Cu) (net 8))
 (segment (start 133.18 79.02) (end 133.18 79.037) (width 0.3048) (layer B.Cu) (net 9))
 (segment (start 133.18 79.037) (end 130.429 80.264) (width 0.3048) (layer B.Cu) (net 9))
 (segment (start 136.78 96.775) (end 136.78 99.35) (width 0.3048) (layer F.Cu) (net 9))
 (segment (start 130.429 90.424) (end 136.78 96.775) (width 0.3048) (layer F.Cu) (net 9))
 (via (at 130.429 90.424) (size 0.6) (drill 0.4) (layers F.Cu B.Cu) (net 9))
 (segment (start 130.429 80.264) (end 130.429 90.424) (width 0.3048) (layer B.Cu) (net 9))
 (segment (start 132.816 79.02) (end 133.18 79.02) (width 0.3048) (layer B.Cu) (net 9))
 (segment (start 133.122 79.02) (end 133.18 79.02) (width 0.3048) (layer B.Cu) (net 9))
 (segment (start 131.252 78.486) (end 132.969 78.486) (width 0.3048) (layer F.Cu) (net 10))
 (segment (start 138.26 76.751) (end 138.26 75.6) (width 0.3048) (layer F.Cu) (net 10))
 (segment (start 136.521802 78.486) (end 138.26 76.751) (width 0.3048) (layer F.Cu) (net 10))
 (segment (start 132.965802 78.486) (end 136.521802 78.486) (width 0.3048) (layer F.Cu) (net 10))
 (segment (start 132.969 78.486) (end 132.965802 78.486) (width 0.3048) (layer F.Cu) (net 10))
 (segment (start 134.62 92.426) (end 133.955 92.426) (width 0.3048) (layer F.Cu) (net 10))
 (segment (start 130.302 79.121) (end 130.937 78.486) (width 0.3048) (layer F.Cu) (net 10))
 (segment (start 130.302 88.773) (end 130.302 79.121) (width 0.3048) (layer F.Cu) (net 10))
 (segment (start 133.955 92.426) (end 130.302 88.773) (width 0.3048) (layer F.Cu) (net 10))
 (segment (start 130.937 78.486) (end 131.252 78.486) (width 0.3048) (layer F.Cu) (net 10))
 (segment (start 136.085 92.426) (end 134.62 92.426) (width 0.3048) (layer F.Cu) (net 10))
 (segment (start 134.62 92.426) (end 134.59 92.426) (width 0.3048) (layer F.Cu) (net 10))
 (segment (start 137.58 99.35) (end 137.58 95.416) (width 0.3048) (layer F.Cu) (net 10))
 (segment (start 136.085 93.921) (end 136.085 92.426) (width 0.3048) (layer F.Cu) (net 10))
 (segment (start 137.58 95.416) (end 136.085 93.921) (width 0.3048) (layer F.Cu) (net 10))
 (segment (start 134.239 91.176) (end 134.229 91.176) (width 0.3048) (layer F.Cu) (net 11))
 (segment (start 134.229 91.176) (end 131.252 88.199) (width 0.3048) (layer F.Cu) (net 11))
 (segment (start 131.252 88.199) (end 131.252 80.645) (width 0.3048) (layer F.Cu) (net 11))
 (segment (start 131.252 80.645) (end 131.572 80.645) (width 0.3048) (layer F.Cu) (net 11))
 (segment (start 131.572 80.645) (end 132.842 79.375) (width 0.3048) (layer F.Cu) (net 11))
 (segment (start 140.8 76.624) (end 140.8 75.6) (width 0.3048) (layer F.Cu) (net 11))
 (segment (start 138.049 79.375) (end 140.8 76.624) (width 0.3048) (layer F.Cu) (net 11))
 (segment (start 132.842 79.375) (end 138.049 79.375) (width 0.3048) (layer F.Cu) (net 11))
 (segment (start 136.085 91.176) (end 134.239 91.176) (width 0.3048) (layer F.Cu) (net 11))
 (segment (start 140.843 75.643) (end 140.8 75.6) (width 0.3048) (layer F.Cu) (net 11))
 (segment (start 138.38 99.35) (end 138.38 94.946) (width 0.3048) (layer F.Cu) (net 11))
 (segment (start 136.642 91.176) (end 136.085 91.176) (width 0.3048) (layer F.Cu) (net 11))
 (segment (start 137.16 91.694) (end 136.642 91.176) (width 0.3048) (layer F.Cu) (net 11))
 (segment (start 137.16 93.726) (end 137.16 91.694) (width 0.3048) (layer F.Cu) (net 11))
 (segment (start 138.38 94.946) (end 137.16 93.726) (width 0.3048) (layer F.Cu) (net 11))
 (segment (start 132.93 100.8) (end 132.169 100.8) (width 0.3048) (layer F.Cu) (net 13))
 (segment (start 132.169 100.8) (end 131.191 99.822) (width 0.3048) (layer F.Cu) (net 13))
 (segment (start 131.191 99.822) (end 131.191 93.345) (width 0.3048) (layer F.Cu) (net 13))
 (segment (start 131.191 93.345) (end 130.429 92.583) (width 0.3048) (layer F.Cu) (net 13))
 (segment (start 130.429 92.583) (end 130.429 91.694) (width 0.3048) (layer F.Cu) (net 13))
 (via (at 130.429 91.694) (size 0.6) (drill 0.4) (layers F.Cu B.Cu) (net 13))
 (segment (start 130.429 91.694) (end 132.207 89.916) (width 0.3048) (layer B.Cu) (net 13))
 (segment (start 132.207 89.916) (end 132.207 87.376) (width 0.3048) (layer B.Cu) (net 13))
 (via (at 132.207 87.376) (size 0.6) (drill 0.4) (layers F.Cu B.Cu) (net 13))
 (segment (start 132.207 87.376) (end 132.715 86.868) (width 0.3048) (layer F.Cu) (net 13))
 (segment (start 132.715 86.868) (end 135.509 86.868) (width 0.3048) (layer F.Cu) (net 13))
 (segment (start 135.509 86.868) (end 136.085 87.444) (width 0.3048) (layer F.Cu) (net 13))
 (segment (start 136.085 87.444) (end 136.085 88.676) (width 0.3048) (layer F.Cu) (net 13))
 (segment (start 134.38 99.35) (end 132.624 99.35) (width 0.3048) (layer F.Cu) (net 32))
 (segment (start 134.757 89.926) (end 136.085 89.926) (width 0.3048) (layer F.Cu) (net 32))
 (segment (start 133.096 88.265) (end 134.757 89.926) (width 0.3048) (layer F.Cu) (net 32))
 (via (at 133.096 88.265) (size 0.6) (drill 0.4) (layers F.Cu B.Cu) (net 32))
 (segment (start 133.096 90.551) (end 133.096 88.265) (width 0.3048) (layer B.Cu) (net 32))
 (segment (start 131.318 92.329) (end 133.096 90.551) (width 0.3048) (layer B.Cu) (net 32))
 (via (at 131.318 92.329) (size 0.6) (drill 0.4) (layers F.Cu B.Cu) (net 32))
 (segment (start 131.826 92.837) (end 131.318 92.329) (width 0.3048) (layer F.Cu) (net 32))
 (segment (start 131.826 98.552) (end 131.826 92.837) (width 0.3048) (layer F.Cu) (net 32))
 (segment (start 132.624 99.35) (end 131.826 98.552) (width 0.3048) (layer F.Cu) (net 32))
 (segment (start 136.085 89.926) (end 134.737 89.926) (width 0.3048) (layer F.Cu) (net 32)))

